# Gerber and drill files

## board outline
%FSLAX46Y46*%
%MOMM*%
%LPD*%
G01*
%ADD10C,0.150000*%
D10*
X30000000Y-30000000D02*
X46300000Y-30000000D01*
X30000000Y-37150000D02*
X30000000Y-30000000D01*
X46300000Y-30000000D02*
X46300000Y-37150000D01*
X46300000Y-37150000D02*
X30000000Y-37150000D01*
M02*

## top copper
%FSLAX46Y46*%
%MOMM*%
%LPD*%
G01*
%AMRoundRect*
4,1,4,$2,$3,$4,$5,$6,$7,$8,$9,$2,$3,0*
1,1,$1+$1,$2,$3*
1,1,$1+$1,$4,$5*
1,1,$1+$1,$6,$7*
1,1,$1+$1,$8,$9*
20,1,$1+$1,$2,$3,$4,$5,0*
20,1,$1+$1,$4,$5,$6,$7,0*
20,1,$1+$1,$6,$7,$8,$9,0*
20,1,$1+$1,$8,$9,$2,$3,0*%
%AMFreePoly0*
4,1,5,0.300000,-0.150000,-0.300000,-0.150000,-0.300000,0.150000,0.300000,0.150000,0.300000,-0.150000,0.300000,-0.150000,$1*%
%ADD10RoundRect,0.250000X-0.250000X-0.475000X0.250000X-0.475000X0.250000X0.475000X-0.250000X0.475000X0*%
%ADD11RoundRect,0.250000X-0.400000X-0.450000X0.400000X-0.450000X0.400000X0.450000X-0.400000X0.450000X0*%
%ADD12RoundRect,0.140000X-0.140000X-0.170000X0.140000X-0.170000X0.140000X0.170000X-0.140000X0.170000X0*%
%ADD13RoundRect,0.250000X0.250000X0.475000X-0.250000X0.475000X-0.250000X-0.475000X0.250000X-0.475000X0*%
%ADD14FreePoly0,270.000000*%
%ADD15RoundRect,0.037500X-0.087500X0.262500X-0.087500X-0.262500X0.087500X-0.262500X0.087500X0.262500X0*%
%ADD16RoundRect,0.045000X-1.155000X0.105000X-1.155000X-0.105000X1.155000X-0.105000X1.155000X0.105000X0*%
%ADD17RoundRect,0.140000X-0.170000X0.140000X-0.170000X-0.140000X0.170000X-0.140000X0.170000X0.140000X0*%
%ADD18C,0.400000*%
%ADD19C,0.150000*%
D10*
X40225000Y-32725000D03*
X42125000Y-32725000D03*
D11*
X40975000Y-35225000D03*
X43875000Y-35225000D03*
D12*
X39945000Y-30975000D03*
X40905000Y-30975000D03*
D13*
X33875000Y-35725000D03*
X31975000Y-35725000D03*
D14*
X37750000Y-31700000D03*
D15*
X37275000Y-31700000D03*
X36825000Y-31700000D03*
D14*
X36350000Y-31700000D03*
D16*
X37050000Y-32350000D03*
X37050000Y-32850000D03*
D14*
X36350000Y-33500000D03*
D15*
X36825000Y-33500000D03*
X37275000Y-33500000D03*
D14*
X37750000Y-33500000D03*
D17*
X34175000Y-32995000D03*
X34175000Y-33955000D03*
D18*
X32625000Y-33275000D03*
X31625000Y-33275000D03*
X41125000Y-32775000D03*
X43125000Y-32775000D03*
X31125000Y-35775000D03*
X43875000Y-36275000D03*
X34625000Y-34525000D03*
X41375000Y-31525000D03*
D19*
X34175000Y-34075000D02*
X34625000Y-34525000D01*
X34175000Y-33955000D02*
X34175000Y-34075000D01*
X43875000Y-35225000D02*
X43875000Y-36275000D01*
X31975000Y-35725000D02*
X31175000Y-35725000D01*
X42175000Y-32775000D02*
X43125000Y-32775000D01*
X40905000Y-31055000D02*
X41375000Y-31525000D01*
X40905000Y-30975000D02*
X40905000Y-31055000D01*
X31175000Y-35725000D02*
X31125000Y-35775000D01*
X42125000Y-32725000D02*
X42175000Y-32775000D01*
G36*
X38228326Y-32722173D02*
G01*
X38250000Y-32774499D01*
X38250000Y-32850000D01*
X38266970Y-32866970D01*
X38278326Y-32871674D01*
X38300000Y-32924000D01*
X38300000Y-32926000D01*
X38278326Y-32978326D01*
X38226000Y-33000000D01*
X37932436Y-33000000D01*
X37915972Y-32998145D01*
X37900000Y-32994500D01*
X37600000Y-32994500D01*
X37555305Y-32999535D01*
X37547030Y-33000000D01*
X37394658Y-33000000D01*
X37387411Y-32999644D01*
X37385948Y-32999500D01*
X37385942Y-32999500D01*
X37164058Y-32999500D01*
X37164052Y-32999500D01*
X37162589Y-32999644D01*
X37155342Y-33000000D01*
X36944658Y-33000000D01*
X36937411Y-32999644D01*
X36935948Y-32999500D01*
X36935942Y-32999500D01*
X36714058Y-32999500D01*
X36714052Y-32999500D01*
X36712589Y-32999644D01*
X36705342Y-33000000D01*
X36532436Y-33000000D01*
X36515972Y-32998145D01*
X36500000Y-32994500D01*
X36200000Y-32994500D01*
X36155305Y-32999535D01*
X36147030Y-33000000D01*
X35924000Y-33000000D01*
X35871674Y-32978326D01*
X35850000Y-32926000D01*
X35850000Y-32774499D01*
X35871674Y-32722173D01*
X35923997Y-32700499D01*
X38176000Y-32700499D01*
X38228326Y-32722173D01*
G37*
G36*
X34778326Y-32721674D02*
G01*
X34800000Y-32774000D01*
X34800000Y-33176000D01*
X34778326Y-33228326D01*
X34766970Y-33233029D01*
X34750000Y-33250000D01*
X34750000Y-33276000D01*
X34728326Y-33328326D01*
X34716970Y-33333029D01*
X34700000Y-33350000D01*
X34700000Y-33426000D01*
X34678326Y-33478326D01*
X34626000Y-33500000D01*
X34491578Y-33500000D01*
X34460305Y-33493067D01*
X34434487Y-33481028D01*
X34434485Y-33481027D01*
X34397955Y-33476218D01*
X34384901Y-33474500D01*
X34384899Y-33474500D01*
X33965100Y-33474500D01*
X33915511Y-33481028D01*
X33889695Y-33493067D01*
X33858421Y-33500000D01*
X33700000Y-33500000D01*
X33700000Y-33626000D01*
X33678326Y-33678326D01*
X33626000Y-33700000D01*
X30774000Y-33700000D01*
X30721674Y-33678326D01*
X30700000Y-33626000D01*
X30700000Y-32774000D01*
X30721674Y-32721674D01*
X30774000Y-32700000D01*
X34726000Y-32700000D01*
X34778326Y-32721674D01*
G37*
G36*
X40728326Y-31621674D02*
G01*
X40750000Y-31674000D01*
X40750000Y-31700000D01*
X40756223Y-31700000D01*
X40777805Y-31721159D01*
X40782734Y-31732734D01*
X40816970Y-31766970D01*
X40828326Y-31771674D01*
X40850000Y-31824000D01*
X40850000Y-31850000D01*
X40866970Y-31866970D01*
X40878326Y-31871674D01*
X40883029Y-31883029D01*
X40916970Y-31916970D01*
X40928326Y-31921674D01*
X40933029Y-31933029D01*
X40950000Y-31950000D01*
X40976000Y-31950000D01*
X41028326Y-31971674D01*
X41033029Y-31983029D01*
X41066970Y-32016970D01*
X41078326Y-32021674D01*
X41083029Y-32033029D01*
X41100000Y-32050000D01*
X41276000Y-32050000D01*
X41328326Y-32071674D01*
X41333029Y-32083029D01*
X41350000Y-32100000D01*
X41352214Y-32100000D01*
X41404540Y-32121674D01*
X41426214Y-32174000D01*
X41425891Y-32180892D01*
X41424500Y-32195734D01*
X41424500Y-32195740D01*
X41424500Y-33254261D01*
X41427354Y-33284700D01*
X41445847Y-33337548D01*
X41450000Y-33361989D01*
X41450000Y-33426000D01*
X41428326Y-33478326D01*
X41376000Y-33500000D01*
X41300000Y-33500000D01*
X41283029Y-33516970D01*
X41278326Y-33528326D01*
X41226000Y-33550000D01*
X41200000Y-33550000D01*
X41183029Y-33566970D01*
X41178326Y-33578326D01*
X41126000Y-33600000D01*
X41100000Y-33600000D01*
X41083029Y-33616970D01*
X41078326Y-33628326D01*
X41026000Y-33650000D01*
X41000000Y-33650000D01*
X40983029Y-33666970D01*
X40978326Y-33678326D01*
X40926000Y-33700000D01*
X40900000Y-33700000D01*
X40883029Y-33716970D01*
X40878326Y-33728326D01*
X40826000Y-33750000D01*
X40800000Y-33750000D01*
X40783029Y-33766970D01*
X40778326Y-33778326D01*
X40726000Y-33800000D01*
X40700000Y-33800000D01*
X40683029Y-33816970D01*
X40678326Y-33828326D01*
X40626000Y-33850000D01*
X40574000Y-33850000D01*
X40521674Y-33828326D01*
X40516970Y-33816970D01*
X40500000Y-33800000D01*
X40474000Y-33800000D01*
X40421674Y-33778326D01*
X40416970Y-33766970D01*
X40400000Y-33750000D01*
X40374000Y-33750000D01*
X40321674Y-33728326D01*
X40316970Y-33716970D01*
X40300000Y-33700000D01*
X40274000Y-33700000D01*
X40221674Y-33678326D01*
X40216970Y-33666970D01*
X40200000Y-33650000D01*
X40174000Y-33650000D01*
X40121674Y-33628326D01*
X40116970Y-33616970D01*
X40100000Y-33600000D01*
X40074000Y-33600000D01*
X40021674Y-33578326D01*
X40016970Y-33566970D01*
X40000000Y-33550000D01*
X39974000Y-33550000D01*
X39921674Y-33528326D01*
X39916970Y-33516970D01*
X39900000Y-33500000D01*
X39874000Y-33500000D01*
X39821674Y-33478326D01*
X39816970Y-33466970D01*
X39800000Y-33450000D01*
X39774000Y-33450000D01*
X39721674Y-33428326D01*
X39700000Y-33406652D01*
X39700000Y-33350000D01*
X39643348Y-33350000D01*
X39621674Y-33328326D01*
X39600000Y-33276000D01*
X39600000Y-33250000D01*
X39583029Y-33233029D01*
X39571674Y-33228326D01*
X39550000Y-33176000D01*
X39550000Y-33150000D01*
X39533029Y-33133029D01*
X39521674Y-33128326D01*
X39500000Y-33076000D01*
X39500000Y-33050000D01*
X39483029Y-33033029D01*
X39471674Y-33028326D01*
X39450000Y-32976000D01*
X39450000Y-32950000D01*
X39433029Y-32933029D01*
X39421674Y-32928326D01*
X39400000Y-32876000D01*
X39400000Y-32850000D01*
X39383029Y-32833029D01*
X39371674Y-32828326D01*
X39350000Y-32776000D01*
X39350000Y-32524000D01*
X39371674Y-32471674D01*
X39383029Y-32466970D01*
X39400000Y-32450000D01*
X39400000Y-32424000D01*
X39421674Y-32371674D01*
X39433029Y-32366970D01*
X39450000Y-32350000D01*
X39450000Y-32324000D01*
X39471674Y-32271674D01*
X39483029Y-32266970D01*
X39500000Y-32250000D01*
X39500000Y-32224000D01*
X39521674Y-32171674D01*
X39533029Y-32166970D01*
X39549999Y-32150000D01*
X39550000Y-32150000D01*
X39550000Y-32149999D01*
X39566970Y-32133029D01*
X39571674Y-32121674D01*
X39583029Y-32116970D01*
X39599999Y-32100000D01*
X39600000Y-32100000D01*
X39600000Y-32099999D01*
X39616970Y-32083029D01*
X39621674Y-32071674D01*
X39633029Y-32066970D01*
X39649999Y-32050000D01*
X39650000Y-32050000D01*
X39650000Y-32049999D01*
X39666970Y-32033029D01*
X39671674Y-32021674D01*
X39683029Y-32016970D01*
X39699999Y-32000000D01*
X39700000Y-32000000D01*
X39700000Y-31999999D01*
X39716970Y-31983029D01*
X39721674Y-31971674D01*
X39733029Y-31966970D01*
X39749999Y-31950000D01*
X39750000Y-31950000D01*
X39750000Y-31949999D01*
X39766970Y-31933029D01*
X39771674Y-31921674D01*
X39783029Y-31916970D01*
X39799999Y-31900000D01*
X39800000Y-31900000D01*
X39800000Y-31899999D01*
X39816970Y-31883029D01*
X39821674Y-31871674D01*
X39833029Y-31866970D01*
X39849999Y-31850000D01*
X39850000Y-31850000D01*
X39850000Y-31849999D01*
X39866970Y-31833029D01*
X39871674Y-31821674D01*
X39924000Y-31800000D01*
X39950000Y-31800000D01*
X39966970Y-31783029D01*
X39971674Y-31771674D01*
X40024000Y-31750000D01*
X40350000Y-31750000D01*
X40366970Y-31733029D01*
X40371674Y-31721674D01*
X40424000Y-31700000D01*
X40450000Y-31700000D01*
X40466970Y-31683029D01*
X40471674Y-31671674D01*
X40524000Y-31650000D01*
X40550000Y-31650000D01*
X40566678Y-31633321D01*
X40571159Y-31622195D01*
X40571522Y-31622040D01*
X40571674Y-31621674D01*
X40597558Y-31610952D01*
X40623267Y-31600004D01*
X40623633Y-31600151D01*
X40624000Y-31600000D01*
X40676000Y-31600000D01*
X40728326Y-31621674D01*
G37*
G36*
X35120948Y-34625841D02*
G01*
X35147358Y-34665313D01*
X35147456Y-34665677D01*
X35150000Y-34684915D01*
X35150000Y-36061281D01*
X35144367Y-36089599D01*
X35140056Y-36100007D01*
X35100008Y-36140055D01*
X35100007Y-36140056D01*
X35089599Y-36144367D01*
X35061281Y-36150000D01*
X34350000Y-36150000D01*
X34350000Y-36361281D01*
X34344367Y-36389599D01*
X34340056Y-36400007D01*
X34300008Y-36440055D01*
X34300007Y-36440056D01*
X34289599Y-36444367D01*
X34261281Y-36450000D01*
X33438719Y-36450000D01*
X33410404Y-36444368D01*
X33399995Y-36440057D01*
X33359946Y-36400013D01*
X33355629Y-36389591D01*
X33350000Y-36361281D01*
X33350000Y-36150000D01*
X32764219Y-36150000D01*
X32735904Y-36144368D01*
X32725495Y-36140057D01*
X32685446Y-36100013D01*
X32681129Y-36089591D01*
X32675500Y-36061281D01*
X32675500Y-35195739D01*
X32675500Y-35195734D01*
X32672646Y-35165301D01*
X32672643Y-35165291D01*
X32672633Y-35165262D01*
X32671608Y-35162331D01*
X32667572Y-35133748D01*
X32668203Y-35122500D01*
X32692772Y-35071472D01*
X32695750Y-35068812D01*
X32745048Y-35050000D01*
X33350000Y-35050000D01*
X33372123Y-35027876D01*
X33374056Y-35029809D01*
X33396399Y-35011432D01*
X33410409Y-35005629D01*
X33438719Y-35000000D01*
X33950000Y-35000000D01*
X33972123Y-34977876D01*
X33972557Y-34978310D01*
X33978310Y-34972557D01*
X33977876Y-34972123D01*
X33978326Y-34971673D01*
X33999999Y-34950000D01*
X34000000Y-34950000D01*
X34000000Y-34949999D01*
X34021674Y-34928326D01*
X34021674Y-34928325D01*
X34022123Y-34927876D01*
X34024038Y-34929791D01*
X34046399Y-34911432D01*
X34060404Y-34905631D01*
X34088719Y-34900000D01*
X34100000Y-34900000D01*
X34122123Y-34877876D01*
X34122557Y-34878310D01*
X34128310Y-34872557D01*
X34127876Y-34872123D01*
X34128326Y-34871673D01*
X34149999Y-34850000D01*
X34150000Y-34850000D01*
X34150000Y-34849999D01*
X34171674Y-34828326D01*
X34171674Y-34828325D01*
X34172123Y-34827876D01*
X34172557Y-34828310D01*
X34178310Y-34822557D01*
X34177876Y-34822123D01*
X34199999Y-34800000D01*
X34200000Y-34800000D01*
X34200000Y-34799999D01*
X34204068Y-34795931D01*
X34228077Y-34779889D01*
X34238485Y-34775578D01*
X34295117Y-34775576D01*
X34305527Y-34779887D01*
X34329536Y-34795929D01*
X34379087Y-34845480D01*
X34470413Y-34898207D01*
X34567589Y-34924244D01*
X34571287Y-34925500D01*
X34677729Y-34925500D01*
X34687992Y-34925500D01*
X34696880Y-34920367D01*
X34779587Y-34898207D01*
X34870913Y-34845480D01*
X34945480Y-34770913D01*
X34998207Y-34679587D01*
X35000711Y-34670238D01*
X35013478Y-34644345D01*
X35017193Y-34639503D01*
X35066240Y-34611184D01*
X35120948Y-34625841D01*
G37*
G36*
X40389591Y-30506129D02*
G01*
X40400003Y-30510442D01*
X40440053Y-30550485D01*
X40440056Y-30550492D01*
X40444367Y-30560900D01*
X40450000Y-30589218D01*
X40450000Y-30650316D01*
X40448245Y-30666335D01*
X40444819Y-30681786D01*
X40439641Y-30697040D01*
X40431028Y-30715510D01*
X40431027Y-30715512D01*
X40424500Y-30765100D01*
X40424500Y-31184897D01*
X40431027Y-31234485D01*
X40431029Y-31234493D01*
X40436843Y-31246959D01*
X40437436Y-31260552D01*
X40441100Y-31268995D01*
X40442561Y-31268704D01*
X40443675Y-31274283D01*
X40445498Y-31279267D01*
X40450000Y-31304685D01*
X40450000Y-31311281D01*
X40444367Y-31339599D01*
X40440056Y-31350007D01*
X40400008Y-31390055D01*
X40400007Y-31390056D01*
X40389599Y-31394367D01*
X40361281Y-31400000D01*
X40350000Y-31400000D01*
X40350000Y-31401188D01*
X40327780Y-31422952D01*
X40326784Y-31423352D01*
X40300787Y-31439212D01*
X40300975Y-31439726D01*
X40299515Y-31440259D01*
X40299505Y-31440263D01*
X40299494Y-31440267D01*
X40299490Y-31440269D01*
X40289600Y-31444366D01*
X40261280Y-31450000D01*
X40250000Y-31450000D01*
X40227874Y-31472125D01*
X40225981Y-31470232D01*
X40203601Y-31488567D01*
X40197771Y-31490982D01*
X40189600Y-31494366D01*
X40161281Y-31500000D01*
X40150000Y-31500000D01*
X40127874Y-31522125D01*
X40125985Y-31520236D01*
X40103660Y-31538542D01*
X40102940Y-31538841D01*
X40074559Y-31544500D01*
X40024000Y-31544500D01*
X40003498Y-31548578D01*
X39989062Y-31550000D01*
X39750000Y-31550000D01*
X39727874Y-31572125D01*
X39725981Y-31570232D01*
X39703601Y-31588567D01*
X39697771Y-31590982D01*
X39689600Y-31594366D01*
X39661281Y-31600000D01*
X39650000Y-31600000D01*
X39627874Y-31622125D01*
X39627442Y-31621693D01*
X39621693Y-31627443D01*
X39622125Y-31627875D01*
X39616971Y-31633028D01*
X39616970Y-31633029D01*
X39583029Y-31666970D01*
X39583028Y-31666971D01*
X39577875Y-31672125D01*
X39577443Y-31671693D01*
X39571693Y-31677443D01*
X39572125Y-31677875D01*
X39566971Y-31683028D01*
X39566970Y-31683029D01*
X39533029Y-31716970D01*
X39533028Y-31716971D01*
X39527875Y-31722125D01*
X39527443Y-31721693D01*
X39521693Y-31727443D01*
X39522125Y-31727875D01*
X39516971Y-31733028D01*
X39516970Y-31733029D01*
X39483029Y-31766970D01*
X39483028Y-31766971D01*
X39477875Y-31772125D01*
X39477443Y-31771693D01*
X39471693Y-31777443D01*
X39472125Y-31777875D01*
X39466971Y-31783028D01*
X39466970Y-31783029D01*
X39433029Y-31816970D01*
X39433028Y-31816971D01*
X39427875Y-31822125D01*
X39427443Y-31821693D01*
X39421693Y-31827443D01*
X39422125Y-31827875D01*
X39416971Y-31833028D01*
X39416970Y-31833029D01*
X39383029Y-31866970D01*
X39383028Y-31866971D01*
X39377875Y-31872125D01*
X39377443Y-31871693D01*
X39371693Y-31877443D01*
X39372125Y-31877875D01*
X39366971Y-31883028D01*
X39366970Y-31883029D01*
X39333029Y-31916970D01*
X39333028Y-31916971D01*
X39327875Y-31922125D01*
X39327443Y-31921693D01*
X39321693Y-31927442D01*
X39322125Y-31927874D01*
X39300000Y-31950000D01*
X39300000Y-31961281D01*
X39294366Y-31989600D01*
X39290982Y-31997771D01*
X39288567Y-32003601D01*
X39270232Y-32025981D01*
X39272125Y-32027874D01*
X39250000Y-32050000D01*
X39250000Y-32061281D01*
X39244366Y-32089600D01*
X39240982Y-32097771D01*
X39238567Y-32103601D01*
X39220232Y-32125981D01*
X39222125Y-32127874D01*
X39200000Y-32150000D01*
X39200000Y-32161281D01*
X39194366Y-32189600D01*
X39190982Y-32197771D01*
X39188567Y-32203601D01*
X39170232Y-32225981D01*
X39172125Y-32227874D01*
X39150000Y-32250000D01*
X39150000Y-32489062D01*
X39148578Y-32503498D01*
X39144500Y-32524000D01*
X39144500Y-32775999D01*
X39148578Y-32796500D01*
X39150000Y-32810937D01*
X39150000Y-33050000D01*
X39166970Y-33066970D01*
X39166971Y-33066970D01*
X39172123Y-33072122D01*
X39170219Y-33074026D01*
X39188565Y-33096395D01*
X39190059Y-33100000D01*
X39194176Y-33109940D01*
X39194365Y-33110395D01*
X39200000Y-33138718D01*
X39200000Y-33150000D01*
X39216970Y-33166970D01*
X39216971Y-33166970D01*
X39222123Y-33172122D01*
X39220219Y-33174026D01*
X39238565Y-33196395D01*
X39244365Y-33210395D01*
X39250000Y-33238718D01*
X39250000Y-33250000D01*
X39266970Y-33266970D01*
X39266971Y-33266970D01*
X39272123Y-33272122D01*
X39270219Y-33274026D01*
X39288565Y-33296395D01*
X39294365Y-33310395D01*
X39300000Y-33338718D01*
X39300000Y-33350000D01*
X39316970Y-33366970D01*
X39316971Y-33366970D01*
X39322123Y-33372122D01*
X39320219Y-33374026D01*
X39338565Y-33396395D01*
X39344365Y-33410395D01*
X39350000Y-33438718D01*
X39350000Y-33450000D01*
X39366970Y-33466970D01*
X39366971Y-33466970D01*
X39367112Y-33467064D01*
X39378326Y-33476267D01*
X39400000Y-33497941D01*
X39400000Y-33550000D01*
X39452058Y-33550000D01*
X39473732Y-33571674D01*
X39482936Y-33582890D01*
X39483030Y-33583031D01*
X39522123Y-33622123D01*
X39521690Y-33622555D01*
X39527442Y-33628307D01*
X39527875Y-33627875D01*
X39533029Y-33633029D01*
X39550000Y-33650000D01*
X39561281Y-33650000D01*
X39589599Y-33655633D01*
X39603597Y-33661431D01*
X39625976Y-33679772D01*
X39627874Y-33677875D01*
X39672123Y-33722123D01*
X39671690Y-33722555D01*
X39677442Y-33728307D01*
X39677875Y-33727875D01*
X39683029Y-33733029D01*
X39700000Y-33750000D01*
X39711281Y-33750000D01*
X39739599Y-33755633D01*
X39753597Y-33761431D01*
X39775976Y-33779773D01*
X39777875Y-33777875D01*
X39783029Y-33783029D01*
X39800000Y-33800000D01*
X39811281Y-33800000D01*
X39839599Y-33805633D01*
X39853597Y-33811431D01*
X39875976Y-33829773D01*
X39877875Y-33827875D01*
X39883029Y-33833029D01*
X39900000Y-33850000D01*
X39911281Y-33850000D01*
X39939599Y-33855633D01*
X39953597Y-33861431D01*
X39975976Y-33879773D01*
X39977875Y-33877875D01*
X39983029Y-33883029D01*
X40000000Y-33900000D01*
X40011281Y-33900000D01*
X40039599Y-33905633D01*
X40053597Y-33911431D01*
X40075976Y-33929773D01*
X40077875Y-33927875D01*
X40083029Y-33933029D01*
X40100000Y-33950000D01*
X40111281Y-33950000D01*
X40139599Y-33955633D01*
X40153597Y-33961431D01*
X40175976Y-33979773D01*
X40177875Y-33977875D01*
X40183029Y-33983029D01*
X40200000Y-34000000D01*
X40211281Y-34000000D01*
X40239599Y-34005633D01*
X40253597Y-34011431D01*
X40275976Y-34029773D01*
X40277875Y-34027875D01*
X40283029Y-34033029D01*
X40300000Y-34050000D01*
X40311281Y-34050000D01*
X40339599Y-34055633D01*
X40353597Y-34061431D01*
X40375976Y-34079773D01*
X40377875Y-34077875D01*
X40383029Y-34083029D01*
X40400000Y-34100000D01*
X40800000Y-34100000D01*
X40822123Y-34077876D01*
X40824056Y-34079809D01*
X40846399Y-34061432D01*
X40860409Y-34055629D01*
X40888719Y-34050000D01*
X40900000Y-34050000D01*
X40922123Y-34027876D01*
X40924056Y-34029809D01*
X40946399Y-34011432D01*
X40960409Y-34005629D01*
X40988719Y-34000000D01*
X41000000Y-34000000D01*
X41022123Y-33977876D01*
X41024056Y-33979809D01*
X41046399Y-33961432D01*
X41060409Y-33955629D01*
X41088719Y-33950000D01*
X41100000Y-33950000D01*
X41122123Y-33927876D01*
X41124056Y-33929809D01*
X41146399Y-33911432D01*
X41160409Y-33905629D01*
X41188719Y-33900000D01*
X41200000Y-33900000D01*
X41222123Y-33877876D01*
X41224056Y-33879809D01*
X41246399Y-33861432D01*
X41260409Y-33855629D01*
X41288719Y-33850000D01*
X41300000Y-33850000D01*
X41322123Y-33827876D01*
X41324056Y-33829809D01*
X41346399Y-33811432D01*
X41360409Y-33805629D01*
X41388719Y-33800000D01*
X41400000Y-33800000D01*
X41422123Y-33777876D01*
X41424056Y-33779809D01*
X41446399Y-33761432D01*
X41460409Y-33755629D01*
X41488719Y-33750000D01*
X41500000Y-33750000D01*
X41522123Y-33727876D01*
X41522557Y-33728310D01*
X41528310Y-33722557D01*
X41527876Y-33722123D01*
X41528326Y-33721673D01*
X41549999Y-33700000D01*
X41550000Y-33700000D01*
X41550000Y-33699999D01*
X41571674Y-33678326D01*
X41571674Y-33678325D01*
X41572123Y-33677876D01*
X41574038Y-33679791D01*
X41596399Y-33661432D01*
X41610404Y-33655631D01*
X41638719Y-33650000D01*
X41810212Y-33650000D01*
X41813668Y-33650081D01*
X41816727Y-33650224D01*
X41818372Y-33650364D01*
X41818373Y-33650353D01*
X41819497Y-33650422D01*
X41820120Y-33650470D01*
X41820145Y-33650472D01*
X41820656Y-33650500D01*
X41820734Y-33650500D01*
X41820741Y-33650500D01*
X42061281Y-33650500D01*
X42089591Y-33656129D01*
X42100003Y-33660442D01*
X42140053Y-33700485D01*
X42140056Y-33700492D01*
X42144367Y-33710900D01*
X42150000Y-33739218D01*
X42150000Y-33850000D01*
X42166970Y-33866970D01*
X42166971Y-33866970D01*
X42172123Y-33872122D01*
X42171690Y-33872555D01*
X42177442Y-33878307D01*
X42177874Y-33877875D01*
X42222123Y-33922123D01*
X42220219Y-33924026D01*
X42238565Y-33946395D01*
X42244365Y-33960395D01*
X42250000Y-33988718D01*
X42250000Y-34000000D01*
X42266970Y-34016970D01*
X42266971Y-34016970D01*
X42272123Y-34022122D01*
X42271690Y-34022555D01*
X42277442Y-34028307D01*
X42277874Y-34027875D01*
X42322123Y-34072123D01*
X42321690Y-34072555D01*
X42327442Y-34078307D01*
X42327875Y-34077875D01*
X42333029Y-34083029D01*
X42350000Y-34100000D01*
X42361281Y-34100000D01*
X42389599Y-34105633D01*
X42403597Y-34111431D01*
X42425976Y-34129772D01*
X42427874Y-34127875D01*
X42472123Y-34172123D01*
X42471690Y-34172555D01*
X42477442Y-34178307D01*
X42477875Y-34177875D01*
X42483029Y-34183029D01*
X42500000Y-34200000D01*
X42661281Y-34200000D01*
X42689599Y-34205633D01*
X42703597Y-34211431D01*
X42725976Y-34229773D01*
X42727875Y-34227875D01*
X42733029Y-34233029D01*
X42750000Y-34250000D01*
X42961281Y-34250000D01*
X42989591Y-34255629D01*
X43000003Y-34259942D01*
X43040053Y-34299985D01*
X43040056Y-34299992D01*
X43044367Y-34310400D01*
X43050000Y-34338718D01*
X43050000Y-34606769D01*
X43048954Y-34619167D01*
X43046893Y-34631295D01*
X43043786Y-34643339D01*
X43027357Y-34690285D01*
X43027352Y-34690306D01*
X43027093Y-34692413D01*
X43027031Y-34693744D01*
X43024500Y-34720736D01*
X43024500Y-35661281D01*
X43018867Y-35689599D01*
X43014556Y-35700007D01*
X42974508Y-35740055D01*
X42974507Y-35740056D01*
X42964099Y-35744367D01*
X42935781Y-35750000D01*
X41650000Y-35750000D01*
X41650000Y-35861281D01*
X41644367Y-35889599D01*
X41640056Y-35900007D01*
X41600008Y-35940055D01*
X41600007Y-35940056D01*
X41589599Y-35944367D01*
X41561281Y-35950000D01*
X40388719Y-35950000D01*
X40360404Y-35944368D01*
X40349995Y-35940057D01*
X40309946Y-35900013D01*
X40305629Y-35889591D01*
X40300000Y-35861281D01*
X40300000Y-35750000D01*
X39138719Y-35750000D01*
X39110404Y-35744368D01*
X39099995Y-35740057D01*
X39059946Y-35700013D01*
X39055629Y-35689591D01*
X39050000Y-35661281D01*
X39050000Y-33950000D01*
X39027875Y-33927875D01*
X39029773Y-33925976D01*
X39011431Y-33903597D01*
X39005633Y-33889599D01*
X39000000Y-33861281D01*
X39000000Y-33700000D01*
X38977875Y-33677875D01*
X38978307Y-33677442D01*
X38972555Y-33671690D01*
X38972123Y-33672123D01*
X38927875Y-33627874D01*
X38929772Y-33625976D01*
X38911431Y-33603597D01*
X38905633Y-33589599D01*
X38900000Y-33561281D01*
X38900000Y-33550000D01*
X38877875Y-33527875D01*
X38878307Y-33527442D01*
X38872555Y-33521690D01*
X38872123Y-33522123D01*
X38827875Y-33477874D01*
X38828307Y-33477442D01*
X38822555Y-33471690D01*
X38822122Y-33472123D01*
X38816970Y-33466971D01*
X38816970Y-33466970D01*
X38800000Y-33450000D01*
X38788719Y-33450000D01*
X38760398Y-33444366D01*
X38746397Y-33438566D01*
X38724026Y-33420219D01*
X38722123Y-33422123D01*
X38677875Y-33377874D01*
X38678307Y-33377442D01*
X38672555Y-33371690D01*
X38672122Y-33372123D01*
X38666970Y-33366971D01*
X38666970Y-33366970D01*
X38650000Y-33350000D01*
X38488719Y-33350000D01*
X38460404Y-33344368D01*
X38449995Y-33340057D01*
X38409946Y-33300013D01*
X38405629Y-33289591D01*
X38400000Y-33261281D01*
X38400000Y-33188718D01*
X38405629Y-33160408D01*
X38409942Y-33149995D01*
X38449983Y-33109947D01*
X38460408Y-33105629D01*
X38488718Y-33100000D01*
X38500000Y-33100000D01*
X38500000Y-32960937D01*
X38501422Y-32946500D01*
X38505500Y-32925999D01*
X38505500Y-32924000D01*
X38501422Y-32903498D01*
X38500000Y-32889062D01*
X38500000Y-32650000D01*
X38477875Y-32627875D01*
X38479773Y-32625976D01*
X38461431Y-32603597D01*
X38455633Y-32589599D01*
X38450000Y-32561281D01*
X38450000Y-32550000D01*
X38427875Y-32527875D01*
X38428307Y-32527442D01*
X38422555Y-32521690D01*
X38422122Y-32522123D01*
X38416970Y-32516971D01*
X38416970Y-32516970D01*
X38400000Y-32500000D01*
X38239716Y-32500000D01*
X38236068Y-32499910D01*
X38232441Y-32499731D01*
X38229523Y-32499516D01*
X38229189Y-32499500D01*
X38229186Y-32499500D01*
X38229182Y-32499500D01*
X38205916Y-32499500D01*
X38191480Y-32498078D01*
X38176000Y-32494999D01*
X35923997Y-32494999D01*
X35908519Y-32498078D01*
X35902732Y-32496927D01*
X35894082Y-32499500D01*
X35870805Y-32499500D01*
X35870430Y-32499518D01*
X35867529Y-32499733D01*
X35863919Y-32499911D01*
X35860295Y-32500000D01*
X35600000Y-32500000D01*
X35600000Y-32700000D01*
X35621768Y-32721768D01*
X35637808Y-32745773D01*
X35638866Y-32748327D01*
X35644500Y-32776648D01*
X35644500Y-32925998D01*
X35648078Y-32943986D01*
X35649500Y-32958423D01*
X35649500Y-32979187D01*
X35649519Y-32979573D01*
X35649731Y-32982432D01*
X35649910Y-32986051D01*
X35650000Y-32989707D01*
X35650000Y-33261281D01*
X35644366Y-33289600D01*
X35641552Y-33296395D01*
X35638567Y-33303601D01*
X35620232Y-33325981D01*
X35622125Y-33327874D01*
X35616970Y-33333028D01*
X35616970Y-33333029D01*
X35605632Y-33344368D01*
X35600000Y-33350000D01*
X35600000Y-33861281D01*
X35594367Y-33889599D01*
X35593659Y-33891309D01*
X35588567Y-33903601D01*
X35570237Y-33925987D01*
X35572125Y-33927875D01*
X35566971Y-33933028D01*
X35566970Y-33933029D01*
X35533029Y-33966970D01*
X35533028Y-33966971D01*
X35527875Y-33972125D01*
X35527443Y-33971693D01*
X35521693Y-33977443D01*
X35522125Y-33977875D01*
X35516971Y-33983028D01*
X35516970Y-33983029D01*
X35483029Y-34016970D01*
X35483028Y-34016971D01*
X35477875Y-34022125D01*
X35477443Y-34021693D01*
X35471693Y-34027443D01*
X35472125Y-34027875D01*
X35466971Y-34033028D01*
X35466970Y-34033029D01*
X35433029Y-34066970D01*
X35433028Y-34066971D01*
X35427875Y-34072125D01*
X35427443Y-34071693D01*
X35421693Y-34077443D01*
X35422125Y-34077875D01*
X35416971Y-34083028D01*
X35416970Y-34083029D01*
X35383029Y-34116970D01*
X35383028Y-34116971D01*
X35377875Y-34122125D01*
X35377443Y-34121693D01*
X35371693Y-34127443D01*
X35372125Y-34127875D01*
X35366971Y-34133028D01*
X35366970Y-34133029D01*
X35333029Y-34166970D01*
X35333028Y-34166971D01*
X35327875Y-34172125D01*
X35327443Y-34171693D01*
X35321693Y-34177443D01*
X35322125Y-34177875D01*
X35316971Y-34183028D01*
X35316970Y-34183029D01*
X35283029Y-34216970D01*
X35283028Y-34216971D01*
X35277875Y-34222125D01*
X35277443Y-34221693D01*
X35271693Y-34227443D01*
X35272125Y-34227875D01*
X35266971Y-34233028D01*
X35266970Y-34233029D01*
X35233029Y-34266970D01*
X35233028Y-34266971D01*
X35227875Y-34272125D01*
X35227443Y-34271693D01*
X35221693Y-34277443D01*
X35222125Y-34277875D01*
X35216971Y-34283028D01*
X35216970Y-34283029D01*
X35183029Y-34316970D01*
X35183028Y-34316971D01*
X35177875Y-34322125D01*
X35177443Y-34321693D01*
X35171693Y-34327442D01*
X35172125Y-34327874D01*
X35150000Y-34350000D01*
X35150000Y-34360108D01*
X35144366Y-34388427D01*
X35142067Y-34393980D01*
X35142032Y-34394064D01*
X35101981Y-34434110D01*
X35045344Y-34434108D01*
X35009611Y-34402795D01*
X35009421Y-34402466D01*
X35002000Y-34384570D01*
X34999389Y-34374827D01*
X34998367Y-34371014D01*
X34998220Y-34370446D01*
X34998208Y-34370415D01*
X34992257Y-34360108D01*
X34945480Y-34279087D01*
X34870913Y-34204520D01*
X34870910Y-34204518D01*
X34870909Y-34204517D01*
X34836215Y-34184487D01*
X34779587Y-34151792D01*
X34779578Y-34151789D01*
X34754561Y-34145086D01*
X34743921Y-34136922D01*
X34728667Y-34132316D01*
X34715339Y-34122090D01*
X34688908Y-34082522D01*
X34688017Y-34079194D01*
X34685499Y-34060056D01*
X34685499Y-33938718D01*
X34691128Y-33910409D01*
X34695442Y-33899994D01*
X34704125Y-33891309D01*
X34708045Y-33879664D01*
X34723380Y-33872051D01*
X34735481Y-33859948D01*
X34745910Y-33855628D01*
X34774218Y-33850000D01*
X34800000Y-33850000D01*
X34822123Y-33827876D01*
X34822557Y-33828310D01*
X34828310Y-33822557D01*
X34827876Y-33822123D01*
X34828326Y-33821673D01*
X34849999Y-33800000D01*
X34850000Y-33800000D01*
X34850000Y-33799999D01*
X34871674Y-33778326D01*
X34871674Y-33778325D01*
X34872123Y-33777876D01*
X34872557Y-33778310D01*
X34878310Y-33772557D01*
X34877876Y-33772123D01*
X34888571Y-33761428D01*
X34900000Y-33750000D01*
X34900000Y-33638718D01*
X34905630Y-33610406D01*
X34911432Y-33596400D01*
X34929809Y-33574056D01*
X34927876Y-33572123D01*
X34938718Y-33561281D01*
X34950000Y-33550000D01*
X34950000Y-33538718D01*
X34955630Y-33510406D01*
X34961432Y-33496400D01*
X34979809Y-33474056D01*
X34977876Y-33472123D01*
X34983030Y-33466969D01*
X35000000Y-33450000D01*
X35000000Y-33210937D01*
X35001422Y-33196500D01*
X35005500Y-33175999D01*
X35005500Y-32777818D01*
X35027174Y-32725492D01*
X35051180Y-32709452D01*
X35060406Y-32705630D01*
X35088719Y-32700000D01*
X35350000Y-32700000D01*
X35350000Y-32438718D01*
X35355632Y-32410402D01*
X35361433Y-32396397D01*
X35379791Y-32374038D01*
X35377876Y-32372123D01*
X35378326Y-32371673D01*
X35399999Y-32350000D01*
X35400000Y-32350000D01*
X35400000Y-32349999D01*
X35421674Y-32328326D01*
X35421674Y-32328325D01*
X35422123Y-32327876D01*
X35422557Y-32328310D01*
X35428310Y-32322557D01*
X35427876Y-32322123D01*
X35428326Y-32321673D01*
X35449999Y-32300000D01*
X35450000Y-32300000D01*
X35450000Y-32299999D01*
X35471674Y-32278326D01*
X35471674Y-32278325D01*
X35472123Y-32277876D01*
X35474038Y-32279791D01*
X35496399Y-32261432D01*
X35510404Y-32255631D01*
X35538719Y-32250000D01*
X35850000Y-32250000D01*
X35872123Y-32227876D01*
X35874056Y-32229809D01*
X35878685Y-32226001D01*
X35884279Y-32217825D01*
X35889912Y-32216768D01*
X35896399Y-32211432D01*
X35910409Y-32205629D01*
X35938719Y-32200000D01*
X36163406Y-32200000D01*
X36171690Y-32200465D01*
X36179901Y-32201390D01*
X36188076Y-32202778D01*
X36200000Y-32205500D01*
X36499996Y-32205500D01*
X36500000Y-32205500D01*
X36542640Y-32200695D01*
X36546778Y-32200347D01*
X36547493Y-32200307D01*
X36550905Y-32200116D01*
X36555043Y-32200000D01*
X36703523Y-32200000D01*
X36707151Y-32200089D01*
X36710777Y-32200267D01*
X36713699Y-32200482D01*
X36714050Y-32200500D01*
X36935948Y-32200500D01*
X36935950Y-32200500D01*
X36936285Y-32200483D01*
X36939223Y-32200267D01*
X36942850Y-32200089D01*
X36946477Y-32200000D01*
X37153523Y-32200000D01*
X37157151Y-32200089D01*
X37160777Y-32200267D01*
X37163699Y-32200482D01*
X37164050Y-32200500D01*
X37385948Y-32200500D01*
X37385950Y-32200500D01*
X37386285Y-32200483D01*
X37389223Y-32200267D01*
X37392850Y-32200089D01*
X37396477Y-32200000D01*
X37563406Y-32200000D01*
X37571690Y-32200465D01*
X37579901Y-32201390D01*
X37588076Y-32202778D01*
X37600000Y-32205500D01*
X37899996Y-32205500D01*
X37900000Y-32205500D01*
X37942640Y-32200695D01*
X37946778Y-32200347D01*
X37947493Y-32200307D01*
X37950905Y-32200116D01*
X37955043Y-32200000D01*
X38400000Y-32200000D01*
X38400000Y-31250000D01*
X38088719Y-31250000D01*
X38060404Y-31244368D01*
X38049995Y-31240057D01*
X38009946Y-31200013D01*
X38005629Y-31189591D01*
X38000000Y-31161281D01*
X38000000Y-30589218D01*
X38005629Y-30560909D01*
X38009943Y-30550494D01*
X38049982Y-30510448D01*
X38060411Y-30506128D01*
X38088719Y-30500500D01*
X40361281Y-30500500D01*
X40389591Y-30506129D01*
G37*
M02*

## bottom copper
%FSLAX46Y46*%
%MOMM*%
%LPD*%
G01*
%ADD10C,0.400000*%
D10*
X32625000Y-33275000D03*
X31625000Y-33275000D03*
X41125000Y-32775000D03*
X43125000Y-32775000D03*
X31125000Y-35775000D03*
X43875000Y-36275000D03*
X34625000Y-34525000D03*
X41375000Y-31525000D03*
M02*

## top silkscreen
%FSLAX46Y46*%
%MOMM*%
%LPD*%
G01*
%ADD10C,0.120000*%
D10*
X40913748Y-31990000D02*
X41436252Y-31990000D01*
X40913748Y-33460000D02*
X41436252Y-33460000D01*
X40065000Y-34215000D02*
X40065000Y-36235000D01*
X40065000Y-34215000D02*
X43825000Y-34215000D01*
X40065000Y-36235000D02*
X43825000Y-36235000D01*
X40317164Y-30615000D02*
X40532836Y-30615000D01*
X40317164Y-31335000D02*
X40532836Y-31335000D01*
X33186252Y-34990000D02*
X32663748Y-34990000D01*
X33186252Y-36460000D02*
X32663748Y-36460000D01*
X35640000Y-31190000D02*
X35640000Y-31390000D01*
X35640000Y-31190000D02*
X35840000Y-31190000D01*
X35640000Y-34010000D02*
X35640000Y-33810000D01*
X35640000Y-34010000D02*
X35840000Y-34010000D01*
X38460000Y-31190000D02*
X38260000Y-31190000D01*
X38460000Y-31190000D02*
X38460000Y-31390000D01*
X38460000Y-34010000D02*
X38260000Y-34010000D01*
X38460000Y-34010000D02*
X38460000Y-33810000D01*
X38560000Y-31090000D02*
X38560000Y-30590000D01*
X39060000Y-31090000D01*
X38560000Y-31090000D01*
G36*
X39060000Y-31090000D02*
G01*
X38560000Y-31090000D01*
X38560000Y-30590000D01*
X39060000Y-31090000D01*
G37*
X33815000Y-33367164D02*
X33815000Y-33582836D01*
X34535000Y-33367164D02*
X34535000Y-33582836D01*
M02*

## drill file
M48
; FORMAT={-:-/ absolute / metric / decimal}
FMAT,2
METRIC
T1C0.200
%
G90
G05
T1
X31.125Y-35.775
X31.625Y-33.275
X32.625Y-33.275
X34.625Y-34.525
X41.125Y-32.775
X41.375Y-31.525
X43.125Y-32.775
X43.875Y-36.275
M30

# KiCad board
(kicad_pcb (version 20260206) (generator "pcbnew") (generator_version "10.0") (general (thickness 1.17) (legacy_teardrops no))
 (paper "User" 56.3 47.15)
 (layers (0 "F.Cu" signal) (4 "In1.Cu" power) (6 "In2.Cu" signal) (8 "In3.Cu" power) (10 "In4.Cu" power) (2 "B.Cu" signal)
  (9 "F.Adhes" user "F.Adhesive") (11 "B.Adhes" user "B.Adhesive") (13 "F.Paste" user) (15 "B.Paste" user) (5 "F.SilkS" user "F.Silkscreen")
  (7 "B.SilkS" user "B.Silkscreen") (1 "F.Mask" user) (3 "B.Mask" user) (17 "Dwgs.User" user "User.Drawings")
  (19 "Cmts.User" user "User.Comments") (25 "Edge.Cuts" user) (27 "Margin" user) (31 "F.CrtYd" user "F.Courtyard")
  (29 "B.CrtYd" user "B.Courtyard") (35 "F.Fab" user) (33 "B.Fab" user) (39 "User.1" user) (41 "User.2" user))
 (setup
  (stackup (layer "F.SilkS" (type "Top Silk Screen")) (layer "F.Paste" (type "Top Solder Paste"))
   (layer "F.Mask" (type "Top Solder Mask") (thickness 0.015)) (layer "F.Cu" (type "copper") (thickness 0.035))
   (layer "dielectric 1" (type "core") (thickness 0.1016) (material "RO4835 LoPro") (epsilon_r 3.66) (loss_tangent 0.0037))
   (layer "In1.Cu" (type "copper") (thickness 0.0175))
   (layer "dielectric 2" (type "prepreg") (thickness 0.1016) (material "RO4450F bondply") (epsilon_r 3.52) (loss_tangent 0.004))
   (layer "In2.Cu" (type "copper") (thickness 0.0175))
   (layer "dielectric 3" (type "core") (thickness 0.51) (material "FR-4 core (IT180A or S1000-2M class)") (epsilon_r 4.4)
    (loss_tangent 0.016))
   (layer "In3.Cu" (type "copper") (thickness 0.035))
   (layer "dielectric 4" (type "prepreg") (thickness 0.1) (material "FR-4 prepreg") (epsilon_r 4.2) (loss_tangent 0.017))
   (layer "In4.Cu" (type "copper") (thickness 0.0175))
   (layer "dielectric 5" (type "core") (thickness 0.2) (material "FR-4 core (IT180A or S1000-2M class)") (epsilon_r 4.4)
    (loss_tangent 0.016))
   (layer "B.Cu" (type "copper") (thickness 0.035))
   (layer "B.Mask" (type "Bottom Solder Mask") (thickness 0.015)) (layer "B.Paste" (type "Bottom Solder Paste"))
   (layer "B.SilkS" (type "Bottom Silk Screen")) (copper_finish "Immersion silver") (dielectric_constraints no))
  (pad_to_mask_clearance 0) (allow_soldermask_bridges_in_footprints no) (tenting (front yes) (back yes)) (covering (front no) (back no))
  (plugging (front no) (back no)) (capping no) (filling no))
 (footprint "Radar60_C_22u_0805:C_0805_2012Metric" (layer "F.Cu") (at 41.175 32.725)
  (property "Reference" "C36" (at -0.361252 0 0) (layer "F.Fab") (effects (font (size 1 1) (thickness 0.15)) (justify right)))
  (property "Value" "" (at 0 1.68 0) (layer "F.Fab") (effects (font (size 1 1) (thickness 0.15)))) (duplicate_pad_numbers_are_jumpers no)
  (fp_line (start -0.261252 -0.735) (end 0.261252 -0.735) (stroke (width 0.12) (type solid)) (layer "F.SilkS"))
  (fp_line (start -0.261252 0.735) (end 0.261252 0.735) (stroke (width 0.12) (type solid)) (layer "F.SilkS"))
  (pad "1" smd roundrect (at -0.95 0) (size 1 1.45) (layers "F.Cu" "F.Mask" "F.Paste") (roundrect_rratio 0.25) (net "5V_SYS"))
  (pad "2" smd roundrect (at 0.95 0) (size 1 1.45) (layers "F.Cu" "F.Mask" "F.Paste") (roundrect_rratio 0.25) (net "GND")))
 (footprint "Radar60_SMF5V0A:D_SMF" (layer "F.Cu") (at 42.425 35.225)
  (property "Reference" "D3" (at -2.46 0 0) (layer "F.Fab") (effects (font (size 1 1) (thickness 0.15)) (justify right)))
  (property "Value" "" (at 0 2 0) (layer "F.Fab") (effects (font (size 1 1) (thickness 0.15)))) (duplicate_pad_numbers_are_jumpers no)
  (fp_line (start -2.36 -1.01) (end -2.36 1.01) (stroke (width 0.12) (type solid)) (layer "F.SilkS"))
  (fp_line (start -2.36 -1.01) (end 1.4 -1.01) (stroke (width 0.12) (type solid)) (layer "F.SilkS"))
  (fp_line (start -2.36 1.01) (end 1.4 1.01) (stroke (width 0.12) (type solid)) (layer "F.SilkS"))
  (pad "1" smd roundrect (at -1.45 0) (size 1.3 1.4) (layers "F.Cu" "F.Mask" "F.Paste") (roundrect_rratio 0.1923077) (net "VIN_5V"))
  (pad "2" smd roundrect (at 1.45 0) (size 1.3 1.4) (layers "F.Cu" "F.Mask" "F.Paste") (roundrect_rratio 0.1923077) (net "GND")))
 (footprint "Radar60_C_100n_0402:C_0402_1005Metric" (layer "F.Cu") (at 40.425 30.975)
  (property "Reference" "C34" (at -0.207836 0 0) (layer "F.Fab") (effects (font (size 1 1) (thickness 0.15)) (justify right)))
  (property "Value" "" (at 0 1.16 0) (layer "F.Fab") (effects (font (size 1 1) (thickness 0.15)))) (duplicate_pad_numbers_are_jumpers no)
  (fp_line (start -0.107836 -0.36) (end 0.107836 -0.36) (stroke (width 0.12) (type solid)) (layer "F.SilkS"))
  (fp_line (start -0.107836 0.36) (end 0.107836 0.36) (stroke (width 0.12) (type solid)) (layer "F.SilkS"))
  (pad "1" smd roundrect (at -0.48 0) (size 0.56 0.62) (layers "F.Cu" "F.Mask" "F.Paste") (roundrect_rratio 0.25) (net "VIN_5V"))
  (pad "2" smd roundrect (at 0.48 0) (size 0.56 0.62) (layers "F.Cu" "F.Mask" "F.Paste") (roundrect_rratio 0.25) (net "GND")))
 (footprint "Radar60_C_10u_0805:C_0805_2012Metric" (layer "F.Cu") (at 32.925 35.725 180)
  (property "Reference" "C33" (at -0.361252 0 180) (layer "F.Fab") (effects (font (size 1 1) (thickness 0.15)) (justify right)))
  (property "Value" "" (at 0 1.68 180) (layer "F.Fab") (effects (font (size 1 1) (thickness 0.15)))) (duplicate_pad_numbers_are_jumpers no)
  (fp_line (start -0.261252 0.735) (end 0.261252 0.735) (stroke (width 0.12) (type solid)) (layer "F.SilkS"))
  (fp_line (start -0.261252 -0.735) (end 0.261252 -0.735) (stroke (width 0.12) (type solid)) (layer "F.SilkS"))
  (pad "1" smd roundrect (at -0.95 0 180) (size 1 1.45) (layers "F.Cu" "F.Mask" "F.Paste") (roundrect_rratio 0.25) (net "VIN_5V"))
  (pad "2" smd roundrect (at 0.95 0 180) (size 1 1.45) (layers "F.Cu" "F.Mask" "F.Paste") (roundrect_rratio 0.25) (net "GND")))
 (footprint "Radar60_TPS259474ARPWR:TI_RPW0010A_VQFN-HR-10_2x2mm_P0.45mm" (layer "F.Cu") (at 37.05 32.6 -90)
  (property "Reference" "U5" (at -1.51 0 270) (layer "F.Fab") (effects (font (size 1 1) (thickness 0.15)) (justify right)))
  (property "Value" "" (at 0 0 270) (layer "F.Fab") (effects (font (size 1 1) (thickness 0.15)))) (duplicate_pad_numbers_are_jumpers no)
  (fp_line (start -1.41 1.41) (end -1.21 1.41) (stroke (width 0.12) (type solid)) (layer "F.SilkS"))
  (fp_line (start -1.41 1.41) (end -1.41 1.21) (stroke (width 0.12) (type solid)) (layer "F.SilkS"))
  (fp_line (start 1.41 1.41) (end 1.21 1.41) (stroke (width 0.12) (type solid)) (layer "F.SilkS"))
  (fp_line (start 1.41 1.41) (end 1.41 1.21) (stroke (width 0.12) (type solid)) (layer "F.SilkS"))
  (fp_line (start -1.41 -1.41) (end -1.41 -1.21) (stroke (width 0.12) (type solid)) (layer "F.SilkS"))
  (fp_line (start -1.41 -1.41) (end -1.21 -1.41) (stroke (width 0.12) (type solid)) (layer "F.SilkS"))
  (fp_line (start 1.41 -1.41) (end 1.41 -1.21) (stroke (width 0.12) (type solid)) (layer "F.SilkS"))
  (fp_line (start 1.41 -1.41) (end 1.21 -1.41) (stroke (width 0.12) (type solid)) (layer "F.SilkS"))
  (fp_poly (pts (xy -1.51 -1.51) (xy -2.01 -1.51) (xy -1.51 -2.01)) (stroke (width 0.12) (type solid)) (fill yes) (layer "F.SilkS"))
  (pad "1" smd custom (at -0.9 -0.7 270) (size 0.6 0.3) (layers "F.Cu" "F.Mask" "F.Paste") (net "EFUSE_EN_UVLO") (solder_mask_margin 0.05)
   (options (clearance outline) (anchor rect)) (primitives))
  (pad "2" smd roundrect (at -0.9 -0.225 270) (size 0.6 0.25) (layers "F.Cu" "F.Mask" "F.Paste") (roundrect_rratio 0.15) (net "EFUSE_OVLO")
   (solder_mask_margin 0.05))
  (pad "3" smd roundrect (at -0.9 0.225 270) (size 0.6 0.25) (layers "F.Cu" "F.Mask" "F.Paste") (roundrect_rratio 0.15) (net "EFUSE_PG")
   (solder_mask_margin 0.05))
  (pad "4" smd custom (at -0.9 0.7 270) (size 0.6 0.3) (layers "F.Cu" "F.Mask" "F.Paste") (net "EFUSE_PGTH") (solder_mask_margin 0.05)
   (options (clearance outline) (anchor rect)) (primitives))
  (pad "5" smd roundrect (at -0.25 0 270) (size 0.3 2.4) (layers "F.Cu" "F.Mask" "F.Paste") (roundrect_rratio 0.15) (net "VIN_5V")
   (solder_mask_margin 0.05))
  (pad "6" smd roundrect (at 0.25 0 270) (size 0.3 2.4) (layers "F.Cu" "F.Mask" "F.Paste") (roundrect_rratio 0.15) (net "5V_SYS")
   (solder_mask_margin 0.05))
  (pad "7" smd custom (at 0.9 0.7 270) (size 0.6 0.3) (layers "F.Cu" "F.Mask" "F.Paste") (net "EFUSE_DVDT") (solder_mask_margin 0.05)
   (options (clearance outline) (anchor rect)) (primitives))
  (pad "8" smd roundrect (at 0.9 0.225 270) (size 0.6 0.25) (layers "F.Cu" "F.Mask" "F.Paste") (roundrect_rratio 0.15) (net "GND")
   (solder_mask_margin 0.05))
  (pad "9" smd roundrect (at 0.9 -0.225 270) (size 0.6 0.25) (layers "F.Cu" "F.Mask" "F.Paste") (roundrect_rratio 0.15) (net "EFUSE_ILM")
   (solder_mask_margin 0.05))
  (pad "10" smd custom (at 0.9 -0.7 270) (size 0.6 0.3) (layers "F.Cu" "F.Mask" "F.Paste") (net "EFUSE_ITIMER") (solder_mask_margin 0.05)
   (options (clearance outline) (anchor rect)) (primitives)))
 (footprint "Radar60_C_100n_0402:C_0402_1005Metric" (layer "F.Cu") (at 34.175 33.475 -90)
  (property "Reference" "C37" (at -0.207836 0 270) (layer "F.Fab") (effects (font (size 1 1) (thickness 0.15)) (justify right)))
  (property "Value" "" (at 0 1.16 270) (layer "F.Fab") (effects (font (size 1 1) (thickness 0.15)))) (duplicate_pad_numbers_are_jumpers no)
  (fp_line (start -0.107836 0.36) (end 0.107836 0.36) (stroke (width 0.12) (type solid)) (layer "F.SilkS"))
  (fp_line (start -0.107836 -0.36) (end 0.107836 -0.36) (stroke (width 0.12) (type solid)) (layer "F.SilkS"))
  (pad "1" smd roundrect (at -0.48 0 270) (size 0.56 0.62) (layers "F.Cu" "F.Mask" "F.Paste") (roundrect_rratio 0.25) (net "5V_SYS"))
  (pad "2" smd roundrect (at 0.48 0 270) (size 0.56 0.62) (layers "F.Cu" "F.Mask" "F.Paste") (roundrect_rratio 0.25) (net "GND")))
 (gr_line (start 30 30) (end 46.3 30) (stroke (width 0.15) (type solid)) (layer "Edge.Cuts"))
 (gr_line (start 30 37.15) (end 30 30) (stroke (width 0.15) (type solid)) (layer "Edge.Cuts"))
 (gr_line (start 46.3 30) (end 46.3 37.15) (stroke (width 0.15) (type solid)) (layer "Edge.Cuts"))
 (gr_line (start 46.3 37.15) (end 30 37.15) (stroke (width 0.15) (type solid)) (layer "Edge.Cuts"))
 (via (at 32.625 33.275) (size 0.4) (drill 0.2) (layers "F.Cu" "B.Cu") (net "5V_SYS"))
 (via (at 31.625 33.275) (size 0.4) (drill 0.2) (layers "F.Cu" "B.Cu") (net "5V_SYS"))
 (via (at 41.125 32.775) (size 0.4) (drill 0.2) (layers "F.Cu" "B.Cu") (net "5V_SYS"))
 (segment (start 34.175 34.075) (end 34.625 34.525) (width 0.15) (layer "F.Cu") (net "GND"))
 (segment (start 34.175 33.955) (end 34.175 34.075) (width 0.15) (layer "F.Cu") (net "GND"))
 (segment (start 43.875 35.225) (end 43.875 36.275) (width 0.15) (layer "F.Cu") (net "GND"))
 (segment (start 31.975 35.725) (end 31.175 35.725) (width 0.15) (layer "F.Cu") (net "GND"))
 (segment (start 42.175 32.775) (end 43.125 32.775) (width 0.15) (layer "F.Cu") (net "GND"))
 (segment (start 40.905 31.055) (end 41.375 31.525) (width 0.15) (layer "F.Cu") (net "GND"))
 (segment (start 40.905 30.975) (end 40.905 31.055) (width 0.15) (layer "F.Cu") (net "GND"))
 (segment (start 31.175 35.725) (end 31.125 35.775) (width 0.15) (layer "F.Cu") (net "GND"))
 (segment (start 42.125 32.725) (end 42.175 32.775) (width 0.15) (layer "F.Cu") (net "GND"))
 (via (at 43.125 32.775) (size 0.4) (drill 0.2) (layers "F.Cu" "B.Cu") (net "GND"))
 (via (at 31.125 35.775) (size 0.4) (drill 0.2) (layers "F.Cu" "B.Cu") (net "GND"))
 (via (at 43.875 36.275) (size 0.4) (drill 0.2) (layers "F.Cu" "B.Cu") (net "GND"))
 (via (at 34.625 34.525) (size 0.4) (drill 0.2) (layers "F.Cu" "B.Cu") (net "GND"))
 (via (at 41.375 31.525) (size 0.4) (drill 0.2) (layers "F.Cu" "B.Cu") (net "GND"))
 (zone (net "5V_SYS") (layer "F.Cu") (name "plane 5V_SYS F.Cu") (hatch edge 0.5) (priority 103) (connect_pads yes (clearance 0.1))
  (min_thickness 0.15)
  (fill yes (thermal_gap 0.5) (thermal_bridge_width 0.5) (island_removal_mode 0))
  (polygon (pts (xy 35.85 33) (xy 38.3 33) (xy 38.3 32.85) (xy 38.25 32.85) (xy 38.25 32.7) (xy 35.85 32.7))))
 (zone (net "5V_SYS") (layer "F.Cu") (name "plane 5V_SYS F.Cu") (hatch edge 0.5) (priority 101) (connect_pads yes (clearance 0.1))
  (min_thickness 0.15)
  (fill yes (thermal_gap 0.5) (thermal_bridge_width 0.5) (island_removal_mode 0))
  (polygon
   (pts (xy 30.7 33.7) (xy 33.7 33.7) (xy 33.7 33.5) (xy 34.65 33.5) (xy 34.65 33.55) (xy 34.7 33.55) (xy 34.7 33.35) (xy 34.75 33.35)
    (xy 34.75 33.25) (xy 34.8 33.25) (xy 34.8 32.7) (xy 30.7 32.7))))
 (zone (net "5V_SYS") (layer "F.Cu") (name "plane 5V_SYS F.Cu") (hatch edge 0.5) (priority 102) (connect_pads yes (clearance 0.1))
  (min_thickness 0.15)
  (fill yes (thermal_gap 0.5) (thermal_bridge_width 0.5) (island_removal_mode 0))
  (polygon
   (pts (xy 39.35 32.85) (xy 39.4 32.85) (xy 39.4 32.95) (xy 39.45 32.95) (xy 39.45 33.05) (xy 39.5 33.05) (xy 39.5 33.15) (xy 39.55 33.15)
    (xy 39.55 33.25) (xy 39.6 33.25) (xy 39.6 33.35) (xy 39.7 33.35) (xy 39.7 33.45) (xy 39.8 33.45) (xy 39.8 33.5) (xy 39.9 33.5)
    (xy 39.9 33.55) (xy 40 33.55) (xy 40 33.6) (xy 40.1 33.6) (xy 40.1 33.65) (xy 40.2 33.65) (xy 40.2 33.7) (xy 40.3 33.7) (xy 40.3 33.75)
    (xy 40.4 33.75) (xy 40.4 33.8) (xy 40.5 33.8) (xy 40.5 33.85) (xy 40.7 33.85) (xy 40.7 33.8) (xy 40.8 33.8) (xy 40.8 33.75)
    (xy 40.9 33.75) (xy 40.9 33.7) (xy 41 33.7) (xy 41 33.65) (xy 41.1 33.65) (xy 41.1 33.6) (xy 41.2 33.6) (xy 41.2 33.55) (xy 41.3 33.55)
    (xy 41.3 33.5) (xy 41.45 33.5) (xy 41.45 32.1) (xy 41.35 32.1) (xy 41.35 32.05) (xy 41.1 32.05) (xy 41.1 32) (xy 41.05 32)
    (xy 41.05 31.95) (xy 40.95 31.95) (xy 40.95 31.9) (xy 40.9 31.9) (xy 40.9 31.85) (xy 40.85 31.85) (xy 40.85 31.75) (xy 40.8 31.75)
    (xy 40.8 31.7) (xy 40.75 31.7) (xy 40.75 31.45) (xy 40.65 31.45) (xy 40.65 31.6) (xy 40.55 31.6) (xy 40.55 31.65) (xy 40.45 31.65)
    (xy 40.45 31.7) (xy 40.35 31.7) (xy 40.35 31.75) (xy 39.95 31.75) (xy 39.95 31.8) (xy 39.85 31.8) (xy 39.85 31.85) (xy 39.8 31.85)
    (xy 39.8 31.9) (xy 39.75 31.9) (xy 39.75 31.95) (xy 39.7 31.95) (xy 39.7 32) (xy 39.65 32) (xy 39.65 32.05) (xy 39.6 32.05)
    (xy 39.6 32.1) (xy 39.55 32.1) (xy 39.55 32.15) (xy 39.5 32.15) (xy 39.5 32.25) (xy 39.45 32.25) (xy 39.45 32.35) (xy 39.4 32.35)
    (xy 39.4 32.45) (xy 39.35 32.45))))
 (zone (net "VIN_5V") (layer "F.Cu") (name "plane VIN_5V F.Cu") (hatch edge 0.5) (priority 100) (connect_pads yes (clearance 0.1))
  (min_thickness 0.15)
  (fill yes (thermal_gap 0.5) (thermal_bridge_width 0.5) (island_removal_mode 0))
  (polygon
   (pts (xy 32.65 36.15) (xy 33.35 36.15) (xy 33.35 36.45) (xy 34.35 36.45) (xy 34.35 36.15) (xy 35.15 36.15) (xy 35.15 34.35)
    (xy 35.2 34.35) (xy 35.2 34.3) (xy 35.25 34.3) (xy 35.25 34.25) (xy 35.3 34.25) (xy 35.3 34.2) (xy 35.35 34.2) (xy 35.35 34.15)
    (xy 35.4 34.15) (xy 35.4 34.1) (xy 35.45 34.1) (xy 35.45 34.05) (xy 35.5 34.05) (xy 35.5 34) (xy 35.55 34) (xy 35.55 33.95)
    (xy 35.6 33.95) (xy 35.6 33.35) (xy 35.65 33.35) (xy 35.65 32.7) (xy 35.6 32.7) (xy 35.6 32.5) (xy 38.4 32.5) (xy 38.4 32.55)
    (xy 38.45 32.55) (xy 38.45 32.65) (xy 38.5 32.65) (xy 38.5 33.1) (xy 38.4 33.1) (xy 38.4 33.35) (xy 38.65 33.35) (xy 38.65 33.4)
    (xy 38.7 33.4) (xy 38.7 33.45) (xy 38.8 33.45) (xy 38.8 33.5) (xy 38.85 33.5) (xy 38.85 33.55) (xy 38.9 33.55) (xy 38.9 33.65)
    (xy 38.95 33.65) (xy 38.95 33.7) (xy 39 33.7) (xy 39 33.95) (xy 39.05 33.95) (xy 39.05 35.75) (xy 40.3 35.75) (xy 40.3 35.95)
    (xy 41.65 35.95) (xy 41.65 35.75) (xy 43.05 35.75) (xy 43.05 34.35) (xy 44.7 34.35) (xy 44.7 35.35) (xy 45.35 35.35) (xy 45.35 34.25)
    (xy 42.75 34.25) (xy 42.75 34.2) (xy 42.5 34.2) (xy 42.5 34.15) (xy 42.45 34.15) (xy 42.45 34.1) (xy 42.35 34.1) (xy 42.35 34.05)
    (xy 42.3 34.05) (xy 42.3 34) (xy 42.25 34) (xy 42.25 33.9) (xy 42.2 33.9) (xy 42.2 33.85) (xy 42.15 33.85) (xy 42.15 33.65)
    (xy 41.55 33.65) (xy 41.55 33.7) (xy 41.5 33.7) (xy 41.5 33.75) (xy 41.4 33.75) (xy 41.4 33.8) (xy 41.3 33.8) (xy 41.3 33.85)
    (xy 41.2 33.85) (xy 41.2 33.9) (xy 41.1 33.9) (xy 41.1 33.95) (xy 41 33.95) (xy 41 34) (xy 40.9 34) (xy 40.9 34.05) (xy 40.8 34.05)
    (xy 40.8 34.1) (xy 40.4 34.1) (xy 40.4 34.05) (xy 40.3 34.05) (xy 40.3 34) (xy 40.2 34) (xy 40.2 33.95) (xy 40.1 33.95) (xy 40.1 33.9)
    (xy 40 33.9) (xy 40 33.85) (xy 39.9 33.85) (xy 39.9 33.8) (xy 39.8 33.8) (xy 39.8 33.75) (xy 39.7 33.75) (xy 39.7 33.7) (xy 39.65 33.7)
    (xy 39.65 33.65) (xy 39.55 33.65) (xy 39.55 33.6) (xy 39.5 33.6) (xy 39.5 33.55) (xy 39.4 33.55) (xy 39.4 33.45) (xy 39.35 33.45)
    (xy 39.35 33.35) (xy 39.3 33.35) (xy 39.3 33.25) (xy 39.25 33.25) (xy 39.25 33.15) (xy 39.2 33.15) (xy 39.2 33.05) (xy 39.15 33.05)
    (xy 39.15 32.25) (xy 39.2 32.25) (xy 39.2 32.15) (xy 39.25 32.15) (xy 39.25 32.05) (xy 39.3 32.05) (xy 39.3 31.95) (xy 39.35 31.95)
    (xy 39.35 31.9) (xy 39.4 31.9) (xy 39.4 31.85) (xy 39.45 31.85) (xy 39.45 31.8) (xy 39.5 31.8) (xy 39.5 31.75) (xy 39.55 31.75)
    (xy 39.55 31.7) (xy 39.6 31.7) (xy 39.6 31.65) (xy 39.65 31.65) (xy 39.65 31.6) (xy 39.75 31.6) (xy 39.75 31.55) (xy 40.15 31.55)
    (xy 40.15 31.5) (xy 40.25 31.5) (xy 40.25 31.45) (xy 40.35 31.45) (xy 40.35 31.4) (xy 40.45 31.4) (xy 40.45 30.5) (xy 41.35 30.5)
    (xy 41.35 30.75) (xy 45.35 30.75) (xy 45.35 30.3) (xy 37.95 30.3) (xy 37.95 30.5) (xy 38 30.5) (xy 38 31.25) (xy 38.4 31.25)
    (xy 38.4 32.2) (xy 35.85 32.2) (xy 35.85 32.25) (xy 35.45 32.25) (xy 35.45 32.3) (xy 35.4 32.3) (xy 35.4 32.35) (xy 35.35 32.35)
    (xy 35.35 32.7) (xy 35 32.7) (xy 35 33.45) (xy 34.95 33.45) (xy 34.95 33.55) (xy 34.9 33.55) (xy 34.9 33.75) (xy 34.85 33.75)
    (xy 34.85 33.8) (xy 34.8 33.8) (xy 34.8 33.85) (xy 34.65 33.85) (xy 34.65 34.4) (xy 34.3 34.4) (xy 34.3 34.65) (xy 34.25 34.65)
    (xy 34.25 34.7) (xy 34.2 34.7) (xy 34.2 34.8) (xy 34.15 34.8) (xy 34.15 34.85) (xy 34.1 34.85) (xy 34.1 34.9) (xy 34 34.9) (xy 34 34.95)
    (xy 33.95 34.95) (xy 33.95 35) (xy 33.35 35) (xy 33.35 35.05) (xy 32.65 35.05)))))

